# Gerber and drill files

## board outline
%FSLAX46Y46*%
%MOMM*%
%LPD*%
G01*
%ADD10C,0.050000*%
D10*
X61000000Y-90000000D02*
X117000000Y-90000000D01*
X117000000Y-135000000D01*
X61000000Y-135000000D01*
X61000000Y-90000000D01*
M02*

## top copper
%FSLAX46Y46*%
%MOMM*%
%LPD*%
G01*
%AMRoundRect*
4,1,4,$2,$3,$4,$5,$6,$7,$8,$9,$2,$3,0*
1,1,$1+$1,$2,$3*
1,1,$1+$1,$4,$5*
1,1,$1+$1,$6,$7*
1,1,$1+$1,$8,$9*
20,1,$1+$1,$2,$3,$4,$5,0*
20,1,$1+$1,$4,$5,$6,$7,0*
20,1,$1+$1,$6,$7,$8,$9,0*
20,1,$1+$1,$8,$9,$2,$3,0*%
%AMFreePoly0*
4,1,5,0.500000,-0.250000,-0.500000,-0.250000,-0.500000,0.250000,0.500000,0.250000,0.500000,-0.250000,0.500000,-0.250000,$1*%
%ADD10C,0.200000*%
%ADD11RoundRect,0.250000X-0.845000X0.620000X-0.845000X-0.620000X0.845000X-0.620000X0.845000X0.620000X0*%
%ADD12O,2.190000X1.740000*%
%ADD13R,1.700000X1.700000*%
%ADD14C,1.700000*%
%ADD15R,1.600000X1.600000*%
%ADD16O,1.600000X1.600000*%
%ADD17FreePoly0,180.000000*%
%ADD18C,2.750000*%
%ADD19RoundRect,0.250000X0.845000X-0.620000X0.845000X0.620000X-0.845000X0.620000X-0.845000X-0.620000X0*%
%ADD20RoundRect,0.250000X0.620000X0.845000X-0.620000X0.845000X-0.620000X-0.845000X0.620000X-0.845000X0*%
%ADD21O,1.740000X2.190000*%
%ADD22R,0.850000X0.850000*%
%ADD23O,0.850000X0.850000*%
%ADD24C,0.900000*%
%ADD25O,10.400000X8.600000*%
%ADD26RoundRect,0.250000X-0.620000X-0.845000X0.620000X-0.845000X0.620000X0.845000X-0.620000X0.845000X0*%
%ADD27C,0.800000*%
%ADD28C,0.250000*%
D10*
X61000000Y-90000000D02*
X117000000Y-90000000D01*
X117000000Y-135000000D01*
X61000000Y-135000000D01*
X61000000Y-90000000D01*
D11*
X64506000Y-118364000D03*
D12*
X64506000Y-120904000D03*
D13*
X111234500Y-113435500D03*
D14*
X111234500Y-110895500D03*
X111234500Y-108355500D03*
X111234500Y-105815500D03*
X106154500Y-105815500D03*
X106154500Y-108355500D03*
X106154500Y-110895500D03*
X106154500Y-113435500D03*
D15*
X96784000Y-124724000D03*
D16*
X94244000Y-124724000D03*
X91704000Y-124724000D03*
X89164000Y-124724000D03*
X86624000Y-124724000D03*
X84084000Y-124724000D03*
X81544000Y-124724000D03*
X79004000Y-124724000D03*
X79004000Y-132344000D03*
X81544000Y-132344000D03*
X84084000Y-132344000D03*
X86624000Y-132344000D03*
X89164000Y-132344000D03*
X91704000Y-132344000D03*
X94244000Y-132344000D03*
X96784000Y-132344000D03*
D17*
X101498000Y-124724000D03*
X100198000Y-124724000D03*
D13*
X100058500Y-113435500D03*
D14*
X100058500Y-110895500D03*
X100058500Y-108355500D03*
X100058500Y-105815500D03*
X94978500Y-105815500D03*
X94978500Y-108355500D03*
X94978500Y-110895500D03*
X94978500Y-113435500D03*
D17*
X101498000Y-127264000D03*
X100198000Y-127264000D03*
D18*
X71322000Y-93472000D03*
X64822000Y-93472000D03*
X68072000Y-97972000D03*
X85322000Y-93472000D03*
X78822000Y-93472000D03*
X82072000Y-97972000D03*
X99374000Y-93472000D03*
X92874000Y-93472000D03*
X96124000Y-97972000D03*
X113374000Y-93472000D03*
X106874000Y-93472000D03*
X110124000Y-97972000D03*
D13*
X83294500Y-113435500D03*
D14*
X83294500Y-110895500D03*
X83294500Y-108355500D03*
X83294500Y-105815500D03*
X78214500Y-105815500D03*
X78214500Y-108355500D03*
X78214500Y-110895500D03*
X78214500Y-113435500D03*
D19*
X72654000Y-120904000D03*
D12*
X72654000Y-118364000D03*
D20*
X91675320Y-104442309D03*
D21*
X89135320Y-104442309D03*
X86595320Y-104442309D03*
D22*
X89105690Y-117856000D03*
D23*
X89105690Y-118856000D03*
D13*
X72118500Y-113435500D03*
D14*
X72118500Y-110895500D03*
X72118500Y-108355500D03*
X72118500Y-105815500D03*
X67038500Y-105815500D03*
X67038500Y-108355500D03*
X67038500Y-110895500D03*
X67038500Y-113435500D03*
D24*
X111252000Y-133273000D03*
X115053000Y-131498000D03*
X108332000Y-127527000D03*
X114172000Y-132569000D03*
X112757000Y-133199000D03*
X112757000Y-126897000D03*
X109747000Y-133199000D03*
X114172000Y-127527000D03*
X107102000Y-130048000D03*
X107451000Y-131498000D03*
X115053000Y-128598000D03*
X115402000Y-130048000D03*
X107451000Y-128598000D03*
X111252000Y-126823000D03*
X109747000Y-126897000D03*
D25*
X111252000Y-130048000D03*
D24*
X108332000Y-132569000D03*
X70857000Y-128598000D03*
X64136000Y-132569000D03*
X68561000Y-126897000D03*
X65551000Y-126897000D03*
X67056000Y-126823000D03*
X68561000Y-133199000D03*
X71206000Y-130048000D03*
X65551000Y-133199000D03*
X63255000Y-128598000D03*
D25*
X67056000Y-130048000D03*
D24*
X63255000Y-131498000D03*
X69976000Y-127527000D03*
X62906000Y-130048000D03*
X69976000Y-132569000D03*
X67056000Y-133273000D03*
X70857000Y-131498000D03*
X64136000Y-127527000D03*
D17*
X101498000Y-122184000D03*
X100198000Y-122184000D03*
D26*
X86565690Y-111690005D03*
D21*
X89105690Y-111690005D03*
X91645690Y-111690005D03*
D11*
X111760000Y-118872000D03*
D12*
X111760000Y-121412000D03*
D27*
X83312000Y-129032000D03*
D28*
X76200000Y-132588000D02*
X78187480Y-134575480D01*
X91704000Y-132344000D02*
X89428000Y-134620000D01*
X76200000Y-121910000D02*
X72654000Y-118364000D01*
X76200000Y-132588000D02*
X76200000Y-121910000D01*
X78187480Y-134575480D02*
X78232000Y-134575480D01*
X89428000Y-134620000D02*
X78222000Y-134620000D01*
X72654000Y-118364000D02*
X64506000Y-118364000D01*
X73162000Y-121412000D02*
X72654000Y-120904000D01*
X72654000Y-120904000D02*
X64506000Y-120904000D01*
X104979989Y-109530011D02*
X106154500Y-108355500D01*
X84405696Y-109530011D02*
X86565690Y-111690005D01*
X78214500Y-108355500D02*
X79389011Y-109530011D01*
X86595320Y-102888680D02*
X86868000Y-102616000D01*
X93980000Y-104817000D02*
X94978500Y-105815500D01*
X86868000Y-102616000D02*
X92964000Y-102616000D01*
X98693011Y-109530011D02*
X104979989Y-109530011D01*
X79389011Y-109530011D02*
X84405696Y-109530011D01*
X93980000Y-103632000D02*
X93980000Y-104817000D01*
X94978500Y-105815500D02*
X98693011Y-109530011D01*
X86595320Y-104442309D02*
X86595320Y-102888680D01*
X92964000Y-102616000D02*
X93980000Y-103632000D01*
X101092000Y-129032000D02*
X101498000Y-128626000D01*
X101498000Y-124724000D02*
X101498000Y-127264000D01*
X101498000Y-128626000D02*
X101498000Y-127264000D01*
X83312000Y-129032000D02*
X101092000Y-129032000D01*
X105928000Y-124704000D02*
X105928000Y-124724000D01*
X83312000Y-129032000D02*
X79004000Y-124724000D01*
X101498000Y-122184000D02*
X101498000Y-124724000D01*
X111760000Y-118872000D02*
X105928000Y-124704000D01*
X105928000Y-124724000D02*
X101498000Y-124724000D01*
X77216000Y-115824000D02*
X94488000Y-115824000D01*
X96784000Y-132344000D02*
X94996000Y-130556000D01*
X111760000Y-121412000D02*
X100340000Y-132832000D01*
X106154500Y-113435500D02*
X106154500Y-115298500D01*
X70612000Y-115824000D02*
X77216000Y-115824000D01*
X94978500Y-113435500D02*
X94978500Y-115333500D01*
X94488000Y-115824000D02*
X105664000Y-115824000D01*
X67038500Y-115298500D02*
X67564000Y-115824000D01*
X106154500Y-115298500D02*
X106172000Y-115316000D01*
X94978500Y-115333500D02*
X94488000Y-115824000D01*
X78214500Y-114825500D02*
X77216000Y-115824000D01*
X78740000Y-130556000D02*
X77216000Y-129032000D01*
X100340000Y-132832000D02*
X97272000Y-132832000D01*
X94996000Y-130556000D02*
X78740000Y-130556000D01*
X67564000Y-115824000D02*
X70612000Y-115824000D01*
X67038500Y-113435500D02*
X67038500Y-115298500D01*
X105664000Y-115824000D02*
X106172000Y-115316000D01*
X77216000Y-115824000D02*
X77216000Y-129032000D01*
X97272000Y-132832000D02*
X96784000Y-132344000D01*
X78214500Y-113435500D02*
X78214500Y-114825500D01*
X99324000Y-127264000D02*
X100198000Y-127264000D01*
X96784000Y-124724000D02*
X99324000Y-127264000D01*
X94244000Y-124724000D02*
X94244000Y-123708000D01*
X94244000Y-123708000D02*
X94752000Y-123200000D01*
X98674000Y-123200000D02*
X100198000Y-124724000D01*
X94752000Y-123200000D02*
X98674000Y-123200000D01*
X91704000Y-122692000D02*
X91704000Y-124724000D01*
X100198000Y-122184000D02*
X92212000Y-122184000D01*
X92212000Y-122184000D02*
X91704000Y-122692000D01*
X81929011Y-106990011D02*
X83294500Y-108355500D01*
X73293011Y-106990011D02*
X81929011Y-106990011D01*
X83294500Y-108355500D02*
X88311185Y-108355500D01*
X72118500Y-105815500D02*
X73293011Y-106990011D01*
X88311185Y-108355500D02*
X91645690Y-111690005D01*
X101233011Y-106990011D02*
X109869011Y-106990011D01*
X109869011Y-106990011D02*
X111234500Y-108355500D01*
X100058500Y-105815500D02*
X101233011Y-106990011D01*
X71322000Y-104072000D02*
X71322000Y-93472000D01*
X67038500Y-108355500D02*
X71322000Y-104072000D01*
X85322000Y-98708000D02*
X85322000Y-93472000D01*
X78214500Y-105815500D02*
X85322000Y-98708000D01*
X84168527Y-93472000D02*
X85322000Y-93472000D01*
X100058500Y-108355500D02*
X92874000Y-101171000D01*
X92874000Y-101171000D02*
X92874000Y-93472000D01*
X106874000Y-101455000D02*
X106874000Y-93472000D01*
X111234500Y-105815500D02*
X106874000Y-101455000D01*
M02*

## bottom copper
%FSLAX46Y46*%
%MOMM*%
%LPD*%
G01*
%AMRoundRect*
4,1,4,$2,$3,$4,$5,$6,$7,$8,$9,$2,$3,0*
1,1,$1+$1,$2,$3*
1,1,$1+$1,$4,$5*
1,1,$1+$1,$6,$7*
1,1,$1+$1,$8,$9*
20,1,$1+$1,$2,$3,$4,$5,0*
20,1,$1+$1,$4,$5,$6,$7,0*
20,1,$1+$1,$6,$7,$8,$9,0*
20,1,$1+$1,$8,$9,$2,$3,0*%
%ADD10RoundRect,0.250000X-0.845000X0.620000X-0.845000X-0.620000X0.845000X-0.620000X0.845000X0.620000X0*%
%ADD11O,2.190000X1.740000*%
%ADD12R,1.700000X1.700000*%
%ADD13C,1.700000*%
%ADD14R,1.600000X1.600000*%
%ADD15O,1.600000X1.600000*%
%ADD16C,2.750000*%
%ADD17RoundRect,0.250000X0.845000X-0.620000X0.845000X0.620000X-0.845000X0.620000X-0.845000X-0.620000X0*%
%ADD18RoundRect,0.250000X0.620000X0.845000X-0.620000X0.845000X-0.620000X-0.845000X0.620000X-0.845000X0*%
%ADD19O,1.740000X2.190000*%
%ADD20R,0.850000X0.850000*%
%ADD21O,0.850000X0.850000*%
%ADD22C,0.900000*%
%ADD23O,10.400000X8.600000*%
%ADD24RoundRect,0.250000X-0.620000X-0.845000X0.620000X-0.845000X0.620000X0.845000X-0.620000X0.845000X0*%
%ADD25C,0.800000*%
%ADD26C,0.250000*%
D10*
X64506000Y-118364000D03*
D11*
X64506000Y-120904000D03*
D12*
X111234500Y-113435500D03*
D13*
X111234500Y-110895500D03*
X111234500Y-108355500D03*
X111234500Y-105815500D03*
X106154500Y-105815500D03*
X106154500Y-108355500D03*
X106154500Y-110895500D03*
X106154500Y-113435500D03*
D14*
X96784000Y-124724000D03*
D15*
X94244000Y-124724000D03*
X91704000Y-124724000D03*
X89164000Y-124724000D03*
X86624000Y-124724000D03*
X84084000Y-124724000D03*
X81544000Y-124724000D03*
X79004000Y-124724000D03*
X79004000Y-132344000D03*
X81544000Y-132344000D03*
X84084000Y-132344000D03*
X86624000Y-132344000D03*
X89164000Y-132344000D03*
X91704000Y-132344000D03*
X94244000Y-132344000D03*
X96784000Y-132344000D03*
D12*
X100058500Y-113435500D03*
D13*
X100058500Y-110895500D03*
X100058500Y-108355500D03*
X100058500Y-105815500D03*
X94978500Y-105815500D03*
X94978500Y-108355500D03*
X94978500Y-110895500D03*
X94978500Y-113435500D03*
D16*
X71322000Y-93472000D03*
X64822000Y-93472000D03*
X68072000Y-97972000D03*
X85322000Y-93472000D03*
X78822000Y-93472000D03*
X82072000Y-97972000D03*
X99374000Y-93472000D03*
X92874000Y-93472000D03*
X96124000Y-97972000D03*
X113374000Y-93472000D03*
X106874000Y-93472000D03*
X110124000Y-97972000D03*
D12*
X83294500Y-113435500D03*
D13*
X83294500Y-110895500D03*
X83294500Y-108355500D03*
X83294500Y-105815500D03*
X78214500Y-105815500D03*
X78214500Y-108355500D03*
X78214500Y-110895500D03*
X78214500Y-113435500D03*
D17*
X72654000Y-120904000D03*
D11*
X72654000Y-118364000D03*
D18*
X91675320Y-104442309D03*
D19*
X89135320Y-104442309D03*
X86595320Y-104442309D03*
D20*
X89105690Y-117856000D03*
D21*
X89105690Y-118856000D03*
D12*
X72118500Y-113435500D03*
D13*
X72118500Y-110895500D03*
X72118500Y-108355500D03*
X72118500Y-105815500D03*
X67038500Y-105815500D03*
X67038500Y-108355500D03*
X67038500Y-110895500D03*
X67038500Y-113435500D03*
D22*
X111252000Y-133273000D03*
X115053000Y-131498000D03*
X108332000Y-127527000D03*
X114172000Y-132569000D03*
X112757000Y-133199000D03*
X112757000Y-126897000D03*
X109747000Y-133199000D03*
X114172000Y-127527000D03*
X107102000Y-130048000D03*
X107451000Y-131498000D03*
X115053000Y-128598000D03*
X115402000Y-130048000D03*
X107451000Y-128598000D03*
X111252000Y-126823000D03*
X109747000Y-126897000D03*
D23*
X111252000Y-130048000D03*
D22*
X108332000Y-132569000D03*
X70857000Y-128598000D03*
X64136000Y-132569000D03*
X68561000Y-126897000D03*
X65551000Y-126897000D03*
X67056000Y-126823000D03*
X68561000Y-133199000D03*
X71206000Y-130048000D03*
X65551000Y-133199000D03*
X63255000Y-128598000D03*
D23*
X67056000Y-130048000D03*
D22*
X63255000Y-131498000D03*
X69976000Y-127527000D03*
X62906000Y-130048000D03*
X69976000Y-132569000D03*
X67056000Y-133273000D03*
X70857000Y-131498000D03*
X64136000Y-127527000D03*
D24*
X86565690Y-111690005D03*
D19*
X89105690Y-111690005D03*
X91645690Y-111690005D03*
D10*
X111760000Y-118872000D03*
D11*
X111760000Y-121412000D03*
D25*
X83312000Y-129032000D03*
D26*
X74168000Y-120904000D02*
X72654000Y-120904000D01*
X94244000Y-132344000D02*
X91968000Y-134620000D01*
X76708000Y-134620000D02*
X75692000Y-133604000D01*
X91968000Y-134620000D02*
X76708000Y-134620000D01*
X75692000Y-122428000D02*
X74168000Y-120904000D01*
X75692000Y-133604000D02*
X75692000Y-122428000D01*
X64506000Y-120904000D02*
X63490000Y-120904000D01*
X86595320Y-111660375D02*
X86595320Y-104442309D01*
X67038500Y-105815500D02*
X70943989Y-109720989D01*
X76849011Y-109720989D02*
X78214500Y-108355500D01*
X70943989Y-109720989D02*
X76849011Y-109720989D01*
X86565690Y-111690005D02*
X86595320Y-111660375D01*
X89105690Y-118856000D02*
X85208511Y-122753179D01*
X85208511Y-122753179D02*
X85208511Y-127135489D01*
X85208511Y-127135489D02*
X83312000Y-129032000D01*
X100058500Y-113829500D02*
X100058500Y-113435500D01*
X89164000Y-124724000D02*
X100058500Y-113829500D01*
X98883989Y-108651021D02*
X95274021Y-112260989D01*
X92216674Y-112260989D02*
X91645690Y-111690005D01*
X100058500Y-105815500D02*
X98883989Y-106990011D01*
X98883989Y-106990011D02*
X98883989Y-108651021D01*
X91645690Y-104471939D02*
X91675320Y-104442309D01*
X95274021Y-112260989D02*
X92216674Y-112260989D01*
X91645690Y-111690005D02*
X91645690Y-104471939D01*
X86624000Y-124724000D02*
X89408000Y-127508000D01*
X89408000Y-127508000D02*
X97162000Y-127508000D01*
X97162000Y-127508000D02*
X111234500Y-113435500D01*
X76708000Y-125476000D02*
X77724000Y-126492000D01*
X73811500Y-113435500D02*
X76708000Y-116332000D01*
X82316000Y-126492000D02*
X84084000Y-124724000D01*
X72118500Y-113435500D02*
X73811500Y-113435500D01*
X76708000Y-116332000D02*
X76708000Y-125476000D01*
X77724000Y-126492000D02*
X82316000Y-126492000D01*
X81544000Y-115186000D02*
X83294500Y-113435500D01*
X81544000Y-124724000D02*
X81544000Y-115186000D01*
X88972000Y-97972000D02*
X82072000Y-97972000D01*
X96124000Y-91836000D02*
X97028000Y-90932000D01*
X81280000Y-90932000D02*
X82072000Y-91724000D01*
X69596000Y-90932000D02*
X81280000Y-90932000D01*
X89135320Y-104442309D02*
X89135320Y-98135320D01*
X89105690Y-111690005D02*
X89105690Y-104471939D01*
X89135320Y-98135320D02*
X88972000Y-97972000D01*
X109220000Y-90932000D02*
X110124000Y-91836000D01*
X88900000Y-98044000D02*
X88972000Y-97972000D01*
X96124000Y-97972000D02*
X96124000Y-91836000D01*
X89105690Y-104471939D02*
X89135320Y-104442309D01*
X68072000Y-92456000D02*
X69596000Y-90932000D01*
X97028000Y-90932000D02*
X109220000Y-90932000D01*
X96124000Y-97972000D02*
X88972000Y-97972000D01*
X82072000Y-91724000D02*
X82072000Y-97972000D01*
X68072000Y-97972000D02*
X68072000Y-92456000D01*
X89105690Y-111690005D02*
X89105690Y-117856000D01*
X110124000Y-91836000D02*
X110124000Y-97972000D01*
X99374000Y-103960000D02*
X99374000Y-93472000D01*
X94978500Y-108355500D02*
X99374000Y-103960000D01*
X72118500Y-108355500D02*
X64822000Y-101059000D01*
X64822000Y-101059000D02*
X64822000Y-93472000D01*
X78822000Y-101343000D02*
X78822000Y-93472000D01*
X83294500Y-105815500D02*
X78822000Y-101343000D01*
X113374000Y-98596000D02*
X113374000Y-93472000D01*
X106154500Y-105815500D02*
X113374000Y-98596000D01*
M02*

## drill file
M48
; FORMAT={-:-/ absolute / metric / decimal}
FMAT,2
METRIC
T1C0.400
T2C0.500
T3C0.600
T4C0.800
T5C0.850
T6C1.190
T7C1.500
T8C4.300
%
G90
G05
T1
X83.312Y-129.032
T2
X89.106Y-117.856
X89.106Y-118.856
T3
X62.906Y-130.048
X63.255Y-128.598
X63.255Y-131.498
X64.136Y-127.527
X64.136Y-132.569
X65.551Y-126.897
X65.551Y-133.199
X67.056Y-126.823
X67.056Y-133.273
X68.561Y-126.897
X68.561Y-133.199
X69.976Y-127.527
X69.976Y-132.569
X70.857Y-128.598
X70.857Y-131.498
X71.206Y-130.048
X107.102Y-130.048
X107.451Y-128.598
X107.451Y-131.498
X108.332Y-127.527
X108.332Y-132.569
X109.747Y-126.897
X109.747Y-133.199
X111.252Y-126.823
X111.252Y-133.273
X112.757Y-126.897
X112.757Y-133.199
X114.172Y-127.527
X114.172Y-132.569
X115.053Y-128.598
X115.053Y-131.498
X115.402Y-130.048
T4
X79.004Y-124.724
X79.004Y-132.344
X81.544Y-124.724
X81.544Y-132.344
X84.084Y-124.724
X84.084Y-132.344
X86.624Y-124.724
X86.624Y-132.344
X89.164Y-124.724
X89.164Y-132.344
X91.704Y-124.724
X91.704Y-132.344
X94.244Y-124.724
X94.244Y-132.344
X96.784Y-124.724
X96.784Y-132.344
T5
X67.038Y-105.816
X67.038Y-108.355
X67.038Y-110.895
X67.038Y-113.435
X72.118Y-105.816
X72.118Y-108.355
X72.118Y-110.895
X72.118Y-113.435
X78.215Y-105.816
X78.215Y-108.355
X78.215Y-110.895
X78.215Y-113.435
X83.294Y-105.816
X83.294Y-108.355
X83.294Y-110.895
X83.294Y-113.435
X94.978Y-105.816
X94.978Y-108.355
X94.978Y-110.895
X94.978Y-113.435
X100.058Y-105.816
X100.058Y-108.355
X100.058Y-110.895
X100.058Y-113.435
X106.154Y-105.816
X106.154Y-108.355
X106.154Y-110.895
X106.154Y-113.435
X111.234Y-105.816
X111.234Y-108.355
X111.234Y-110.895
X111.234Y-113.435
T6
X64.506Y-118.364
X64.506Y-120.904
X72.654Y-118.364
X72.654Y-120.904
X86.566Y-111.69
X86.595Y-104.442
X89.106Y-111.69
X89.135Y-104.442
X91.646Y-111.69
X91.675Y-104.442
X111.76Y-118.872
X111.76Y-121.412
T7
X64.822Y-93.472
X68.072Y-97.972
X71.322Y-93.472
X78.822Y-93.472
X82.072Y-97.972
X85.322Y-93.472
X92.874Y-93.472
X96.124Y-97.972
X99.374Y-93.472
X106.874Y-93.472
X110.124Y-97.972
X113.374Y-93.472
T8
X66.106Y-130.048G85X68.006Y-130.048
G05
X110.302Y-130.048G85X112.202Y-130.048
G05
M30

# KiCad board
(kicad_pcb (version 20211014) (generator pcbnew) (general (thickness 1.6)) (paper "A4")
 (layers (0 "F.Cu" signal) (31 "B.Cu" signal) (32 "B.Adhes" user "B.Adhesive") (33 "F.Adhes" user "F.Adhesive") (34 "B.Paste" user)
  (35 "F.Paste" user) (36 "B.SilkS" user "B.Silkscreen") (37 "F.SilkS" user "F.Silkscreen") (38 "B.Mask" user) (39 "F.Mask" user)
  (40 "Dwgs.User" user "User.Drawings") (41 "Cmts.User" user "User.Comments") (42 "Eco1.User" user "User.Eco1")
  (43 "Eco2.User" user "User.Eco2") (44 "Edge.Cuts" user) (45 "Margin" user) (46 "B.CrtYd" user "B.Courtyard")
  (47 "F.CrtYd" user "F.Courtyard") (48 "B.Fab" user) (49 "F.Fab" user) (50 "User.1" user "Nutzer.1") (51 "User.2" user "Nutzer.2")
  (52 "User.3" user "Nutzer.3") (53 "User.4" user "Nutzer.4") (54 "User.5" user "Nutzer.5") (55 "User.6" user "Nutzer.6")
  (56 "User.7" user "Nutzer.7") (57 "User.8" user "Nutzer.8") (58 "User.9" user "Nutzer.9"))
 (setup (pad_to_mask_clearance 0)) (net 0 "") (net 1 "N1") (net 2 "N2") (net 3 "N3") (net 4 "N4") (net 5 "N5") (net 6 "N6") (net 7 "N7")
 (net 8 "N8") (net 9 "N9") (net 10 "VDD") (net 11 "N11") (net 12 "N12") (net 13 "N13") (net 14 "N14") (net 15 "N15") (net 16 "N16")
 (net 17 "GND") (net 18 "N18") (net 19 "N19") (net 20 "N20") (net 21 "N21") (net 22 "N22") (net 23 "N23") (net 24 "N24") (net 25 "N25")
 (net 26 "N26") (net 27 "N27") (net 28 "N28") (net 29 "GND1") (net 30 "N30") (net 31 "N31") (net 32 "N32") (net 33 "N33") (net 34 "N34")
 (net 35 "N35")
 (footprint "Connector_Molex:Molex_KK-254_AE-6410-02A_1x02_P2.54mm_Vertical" (layer "F.Cu") (at 64.506 118.364 -90)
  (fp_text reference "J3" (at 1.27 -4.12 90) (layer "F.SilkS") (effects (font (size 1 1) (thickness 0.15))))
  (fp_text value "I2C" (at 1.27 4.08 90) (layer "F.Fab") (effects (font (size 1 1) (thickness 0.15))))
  (pad "1" thru_hole roundrect (at 0 0 270) (size 1.74 2.19) (drill 1.19) (layers *.Cu *.Mask) (roundrect_rratio 0.143678) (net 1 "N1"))
  (pad "2" thru_hole oval (at 2.54 0 270) (size 1.74 2.19) (drill 1.19) (layers *.Cu *.Mask) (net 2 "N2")))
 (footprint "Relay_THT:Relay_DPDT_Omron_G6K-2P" (layer "F.Cu") (at 111.2345 113.4355 180)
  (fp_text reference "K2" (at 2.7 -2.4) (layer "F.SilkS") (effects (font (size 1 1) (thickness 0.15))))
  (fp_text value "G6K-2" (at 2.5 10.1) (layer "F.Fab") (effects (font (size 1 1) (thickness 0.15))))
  (pad "1" thru_hole rect (at 0 0 180) (size 1.7 1.7) (drill 0.85) (layers *.Cu *.Mask) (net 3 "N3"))
  (pad "2" thru_hole circle (at 0 2.54 180) (size 1.7 1.7) (drill 0.85) (layers *.Cu *.Mask) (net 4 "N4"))
  (pad "3" thru_hole circle (at 0 5.08 180) (size 1.7 1.7) (drill 0.85) (layers *.Cu *.Mask) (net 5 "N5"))
  (pad "4" thru_hole circle (at 0 7.62 180) (size 1.7 1.7) (drill 0.85) (layers *.Cu *.Mask) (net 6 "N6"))
  (pad "5" thru_hole circle (at 5.08 7.62 180) (size 1.7 1.7) (drill 0.85) (layers *.Cu *.Mask) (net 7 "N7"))
  (pad "6" thru_hole circle (at 5.08 5.08 180) (size 1.7 1.7) (drill 0.85) (layers *.Cu *.Mask) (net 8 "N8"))
  (pad "7" thru_hole circle (at 5.08 2.54 180) (size 1.7 1.7) (drill 0.85) (layers *.Cu *.Mask) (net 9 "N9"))
  (pad "8" thru_hole circle (at 5.08 0 180) (size 1.7 1.7) (drill 0.85) (layers *.Cu *.Mask) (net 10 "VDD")))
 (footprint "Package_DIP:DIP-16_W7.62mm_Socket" (layer "F.Cu") (at 96.784 124.724 -90)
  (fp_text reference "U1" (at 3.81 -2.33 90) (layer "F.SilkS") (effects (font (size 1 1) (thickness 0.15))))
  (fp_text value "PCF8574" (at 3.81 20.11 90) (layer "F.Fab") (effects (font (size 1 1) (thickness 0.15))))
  (pad "1" thru_hole rect (at 0 0 270) (size 1.6 1.6) (drill 0.8) (layers *.Cu *.Mask) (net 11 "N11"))
  (pad "2" thru_hole oval (at 0 2.54 270) (size 1.6 1.6) (drill 0.8) (layers *.Cu *.Mask) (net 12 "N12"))
  (pad "3" thru_hole oval (at 0 5.08 270) (size 1.6 1.6) (drill 0.8) (layers *.Cu *.Mask) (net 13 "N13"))
  (pad "4" thru_hole oval (at 0 7.62 270) (size 1.6 1.6) (drill 0.8) (layers *.Cu *.Mask) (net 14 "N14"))
  (pad "5" thru_hole oval (at 0 10.16 270) (size 1.6 1.6) (drill 0.8) (layers *.Cu *.Mask) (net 3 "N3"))
  (pad "6" thru_hole oval (at 0 12.7 270) (size 1.6 1.6) (drill 0.8) (layers *.Cu *.Mask) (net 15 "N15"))
  (pad "7" thru_hole oval (at 0 15.24 270) (size 1.6 1.6) (drill 0.8) (layers *.Cu *.Mask) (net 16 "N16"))
  (pad "8" thru_hole oval (at 0 17.78 270) (size 1.6 1.6) (drill 0.8) (layers *.Cu *.Mask) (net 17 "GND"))
  (pad "9" thru_hole oval (at 7.62 17.78 270) (size 1.6 1.6) (drill 0.8) (layers *.Cu *.Mask) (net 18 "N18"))
  (pad "10" thru_hole oval (at 7.62 15.24 270) (size 1.6 1.6) (drill 0.8) (layers *.Cu *.Mask) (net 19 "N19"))
  (pad "11" thru_hole oval (at 7.62 12.7 270) (size 1.6 1.6) (drill 0.8) (layers *.Cu *.Mask) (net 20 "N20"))
  (pad "12" thru_hole oval (at 7.62 10.16 270) (size 1.6 1.6) (drill 0.8) (layers *.Cu *.Mask) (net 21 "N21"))
  (pad "13" thru_hole oval (at 7.62 7.62 270) (size 1.6 1.6) (drill 0.8) (layers *.Cu *.Mask) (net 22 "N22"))
  (pad "14" thru_hole oval (at 7.62 5.08 270) (size 1.6 1.6) (drill 0.8) (layers *.Cu *.Mask) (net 1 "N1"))
  (pad "15" thru_hole oval (at 7.62 2.54 270) (size 1.6 1.6) (drill 0.8) (layers *.Cu *.Mask) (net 2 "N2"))
  (pad "16" thru_hole oval (at 7.62 0 270) (size 1.6 1.6) (drill 0.8) (layers *.Cu *.Mask) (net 10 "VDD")))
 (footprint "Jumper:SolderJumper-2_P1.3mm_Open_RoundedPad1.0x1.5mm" (layer "F.Cu") (at 100.848 124.724 180)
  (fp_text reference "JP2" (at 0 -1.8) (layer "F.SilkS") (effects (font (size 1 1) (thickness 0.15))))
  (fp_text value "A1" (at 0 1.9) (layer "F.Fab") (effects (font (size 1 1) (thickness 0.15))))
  (pad "1" smd custom (at -0.65 0 180) (size 1 0.5) (layers "F.Cu" "F.Mask") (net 17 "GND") (zone_connect 2)
   (options (clearance outline) (anchor rect)) (primitives))
  (pad "2" smd custom (at 0.65 0 180) (size 1 0.5) (layers "F.Cu" "F.Mask") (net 12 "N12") (zone_connect 2)
   (options (clearance outline) (anchor rect)) (primitives)))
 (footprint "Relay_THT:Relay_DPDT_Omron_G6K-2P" (layer "F.Cu") (at 100.0585 113.4355 180)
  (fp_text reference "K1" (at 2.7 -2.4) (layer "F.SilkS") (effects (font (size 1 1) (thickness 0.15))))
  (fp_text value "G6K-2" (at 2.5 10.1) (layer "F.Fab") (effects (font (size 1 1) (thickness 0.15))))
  (pad "1" thru_hole rect (at 0 0 180) (size 1.7 1.7) (drill 0.85) (layers *.Cu *.Mask) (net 14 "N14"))
  (pad "2" thru_hole circle (at 0 2.54 180) (size 1.7 1.7) (drill 0.85) (layers *.Cu *.Mask) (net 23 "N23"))
  (pad "3" thru_hole circle (at 0 5.08 180) (size 1.7 1.7) (drill 0.85) (layers *.Cu *.Mask) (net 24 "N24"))
  (pad "4" thru_hole circle (at 0 7.62 180) (size 1.7 1.7) (drill 0.85) (layers *.Cu *.Mask) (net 5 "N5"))
  (pad "5" thru_hole circle (at 5.08 7.62 180) (size 1.7 1.7) (drill 0.85) (layers *.Cu *.Mask) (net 8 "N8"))
  (pad "6" thru_hole circle (at 5.08 5.08 180) (size 1.7 1.7) (drill 0.85) (layers *.Cu *.Mask) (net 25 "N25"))
  (pad "7" thru_hole circle (at 5.08 2.54 180) (size 1.7 1.7) (drill 0.85) (layers *.Cu *.Mask) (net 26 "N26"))
  (pad "8" thru_hole circle (at 5.08 0 180) (size 1.7 1.7) (drill 0.85) (layers *.Cu *.Mask) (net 10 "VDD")))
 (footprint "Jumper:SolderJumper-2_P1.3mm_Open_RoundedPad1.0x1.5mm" (layer "F.Cu") (at 100.848 127.264 180)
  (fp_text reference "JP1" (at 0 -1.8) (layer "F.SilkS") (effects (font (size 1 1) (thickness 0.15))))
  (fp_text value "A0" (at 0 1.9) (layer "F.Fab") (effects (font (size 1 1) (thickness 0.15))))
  (pad "1" smd custom (at -0.65 0 180) (size 1 0.5) (layers "F.Cu" "F.Mask") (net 17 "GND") (zone_connect 2)
   (options (clearance outline) (anchor rect)) (primitives))
  (pad "2" smd custom (at 0.65 0 180) (size 1 0.5) (layers "F.Cu" "F.Mask") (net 11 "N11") (zone_connect 2)
   (options (clearance outline) (anchor rect)) (primitives)))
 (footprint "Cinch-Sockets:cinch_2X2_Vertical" (layer "F.Cu") (at 68.072 93.472)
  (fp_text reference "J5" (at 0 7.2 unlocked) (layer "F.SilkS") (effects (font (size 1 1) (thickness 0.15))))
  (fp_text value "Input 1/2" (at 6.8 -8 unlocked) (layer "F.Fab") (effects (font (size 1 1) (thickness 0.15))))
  (pad "1" thru_hole circle (at 3.25 0) (size 2.75 2.75) (drill 1.5) (layers *.Cu *.Mask) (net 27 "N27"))
  (pad "2" thru_hole circle (at -3.25 0) (size 2.75 2.75) (drill 1.5) (layers *.Cu *.Mask) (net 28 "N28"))
  (pad "3" thru_hole circle (at 0 4.5) (size 2.75 2.75) (drill 1.5) (layers *.Cu *.Mask) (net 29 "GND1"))
  (pad "4" thru_hole circle (at 17.25 0) (size 2.75 2.75) (drill 1.5) (layers *.Cu *.Mask) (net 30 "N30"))
  (pad "5" thru_hole circle (at 10.75 0) (size 2.75 2.75) (drill 1.5) (layers *.Cu *.Mask) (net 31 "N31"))
  (pad "6" thru_hole circle (at 14 4.5) (size 2.75 2.75) (drill 1.5) (layers *.Cu *.Mask) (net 29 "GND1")))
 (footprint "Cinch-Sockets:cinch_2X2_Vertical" (layer "F.Cu") (at 96.124 93.472)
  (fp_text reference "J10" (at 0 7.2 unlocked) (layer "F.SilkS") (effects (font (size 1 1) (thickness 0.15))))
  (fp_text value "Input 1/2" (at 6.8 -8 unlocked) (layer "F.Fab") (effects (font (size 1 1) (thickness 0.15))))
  (pad "1" thru_hole circle (at 3.25 0) (size 2.75 2.75) (drill 1.5) (layers *.Cu *.Mask) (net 25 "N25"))
  (pad "2" thru_hole circle (at -3.25 0) (size 2.75 2.75) (drill 1.5) (layers *.Cu *.Mask) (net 24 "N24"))
  (pad "3" thru_hole circle (at 0 4.5) (size 2.75 2.75) (drill 1.5) (layers *.Cu *.Mask) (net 29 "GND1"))
  (pad "4" thru_hole circle (at 17.25 0) (size 2.75 2.75) (drill 1.5) (layers *.Cu *.Mask) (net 7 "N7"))
  (pad "5" thru_hole circle (at 10.75 0) (size 2.75 2.75) (drill 1.5) (layers *.Cu *.Mask) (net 6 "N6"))
  (pad "6" thru_hole circle (at 14 4.5) (size 2.75 2.75) (drill 1.5) (layers *.Cu *.Mask) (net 29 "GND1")))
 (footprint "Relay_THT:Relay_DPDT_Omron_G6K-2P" (layer "F.Cu") (at 83.2945 113.4355 180)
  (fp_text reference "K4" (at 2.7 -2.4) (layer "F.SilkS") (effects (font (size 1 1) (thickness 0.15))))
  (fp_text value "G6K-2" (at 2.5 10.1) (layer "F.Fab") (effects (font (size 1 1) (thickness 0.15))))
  (pad "1" thru_hole rect (at 0 0 180) (size 1.7 1.7) (drill 0.85) (layers *.Cu *.Mask) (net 16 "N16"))
  (pad "2" thru_hole circle (at 0 2.54 180) (size 1.7 1.7) (drill 0.85) (layers *.Cu *.Mask) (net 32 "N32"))
  (pad "3" thru_hole circle (at 0 5.08 180) (size 1.7 1.7) (drill 0.85) (layers *.Cu *.Mask) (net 5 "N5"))
  (pad "4" thru_hole circle (at 0 7.62 180) (size 1.7 1.7) (drill 0.85) (layers *.Cu *.Mask) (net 31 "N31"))
  (pad "5" thru_hole circle (at 5.08 7.62 180) (size 1.7 1.7) (drill 0.85) (layers *.Cu *.Mask) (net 30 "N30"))
  (pad "6" thru_hole circle (at 5.08 5.08 180) (size 1.7 1.7) (drill 0.85) (layers *.Cu *.Mask) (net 8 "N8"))
  (pad "7" thru_hole circle (at 5.08 2.54 180) (size 1.7 1.7) (drill 0.85) (layers *.Cu *.Mask) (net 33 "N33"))
  (pad "8" thru_hole circle (at 5.08 0 180) (size 1.7 1.7) (drill 0.85) (layers *.Cu *.Mask) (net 10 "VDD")))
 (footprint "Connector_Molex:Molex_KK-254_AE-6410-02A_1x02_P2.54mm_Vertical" (layer "F.Cu") (at 72.654 120.904 90)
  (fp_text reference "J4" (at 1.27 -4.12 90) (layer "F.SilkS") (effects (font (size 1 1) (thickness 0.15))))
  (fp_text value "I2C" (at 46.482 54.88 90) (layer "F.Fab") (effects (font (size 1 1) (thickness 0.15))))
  (pad "1" thru_hole roundrect (at 0 0 90) (size 1.74 2.19) (drill 1.19) (layers *.Cu *.Mask) (roundrect_rratio 0.143678) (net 2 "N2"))
  (pad "2" thru_hole oval (at 2.54 0 90) (size 1.74 2.19) (drill 1.19) (layers *.Cu *.Mask) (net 1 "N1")))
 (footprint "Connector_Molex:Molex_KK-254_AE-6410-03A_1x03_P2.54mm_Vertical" (layer "F.Cu") (at 91.67532 104.442309 180)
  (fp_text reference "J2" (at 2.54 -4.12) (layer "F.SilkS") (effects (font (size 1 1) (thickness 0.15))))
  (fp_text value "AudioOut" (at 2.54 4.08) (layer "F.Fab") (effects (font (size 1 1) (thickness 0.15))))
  (pad "1" thru_hole roundrect (at 0 0 180) (size 1.74 2.19) (drill 1.19) (layers *.Cu *.Mask) (roundrect_rratio 0.143678) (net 5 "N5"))
  (pad "2" thru_hole oval (at 2.54 0 180) (size 1.74 2.19) (drill 1.19) (layers *.Cu *.Mask) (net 29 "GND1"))
  (pad "3" thru_hole oval (at 5.08 0 180) (size 1.74 2.19) (drill 1.19) (layers *.Cu *.Mask) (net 8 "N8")))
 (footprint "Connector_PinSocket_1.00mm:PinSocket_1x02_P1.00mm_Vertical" (layer "F.Cu") (at 89.10569 117.856)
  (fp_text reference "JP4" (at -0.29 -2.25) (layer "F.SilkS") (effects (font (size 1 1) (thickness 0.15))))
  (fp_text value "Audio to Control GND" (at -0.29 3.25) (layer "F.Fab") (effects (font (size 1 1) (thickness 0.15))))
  (pad "1" thru_hole rect (at 0 0) (size 0.85 0.85) (drill 0.5) (layers *.Cu *.Mask) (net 29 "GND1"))
  (pad "2" thru_hole oval (at 0 1) (size 0.85 0.85) (drill 0.5) (layers *.Cu *.Mask) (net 17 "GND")))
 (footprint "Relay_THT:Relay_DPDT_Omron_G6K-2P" (layer "F.Cu") (at 72.1185 113.4355 180)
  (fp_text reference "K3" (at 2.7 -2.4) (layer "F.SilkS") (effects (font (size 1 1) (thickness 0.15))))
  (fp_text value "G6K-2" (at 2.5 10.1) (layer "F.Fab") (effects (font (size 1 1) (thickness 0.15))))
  (pad "1" thru_hole rect (at 0 0 180) (size 1.7 1.7) (drill 0.85) (layers *.Cu *.Mask) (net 15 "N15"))
  (pad "2" thru_hole circle (at 0 2.54 180) (size 1.7 1.7) (drill 0.85) (layers *.Cu *.Mask) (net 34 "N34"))
  (pad "3" thru_hole circle (at 0 5.08 180) (size 1.7 1.7) (drill 0.85) (layers *.Cu *.Mask) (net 28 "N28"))
  (pad "4" thru_hole circle (at 0 7.62 180) (size 1.7 1.7) (drill 0.85) (layers *.Cu *.Mask) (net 5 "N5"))
  (pad "5" thru_hole circle (at 5.08 7.62 180) (size 1.7 1.7) (drill 0.85) (layers *.Cu *.Mask) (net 8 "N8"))
  (pad "6" thru_hole circle (at 5.08 5.08 180) (size 1.7 1.7) (drill 0.85) (layers *.Cu *.Mask) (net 27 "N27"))
  (pad "7" thru_hole circle (at 5.08 2.54 180) (size 1.7 1.7) (drill 0.85) (layers *.Cu *.Mask) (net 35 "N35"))
  (pad "8" thru_hole circle (at 5.08 0 180) (size 1.7 1.7) (drill 0.85) (layers *.Cu *.Mask) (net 10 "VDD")))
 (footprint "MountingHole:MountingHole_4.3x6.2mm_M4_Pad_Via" (layer "F.Cu") (at 111.252 130.048)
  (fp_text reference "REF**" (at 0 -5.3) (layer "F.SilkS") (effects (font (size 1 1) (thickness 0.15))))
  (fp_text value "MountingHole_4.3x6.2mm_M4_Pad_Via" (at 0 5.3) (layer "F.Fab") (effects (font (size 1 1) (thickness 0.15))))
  (pad "1" thru_hole circle (at 0 3.225) (size 0.9 0.9) (drill 0.6) (layers *.Cu *.Mask))
  (pad "1" thru_hole circle (at 3.801 1.45) (size 0.9 0.9) (drill 0.6) (layers *.Cu *.Mask))
  (pad "1" thru_hole circle (at -2.92 -2.521) (size 0.9 0.9) (drill 0.6) (layers *.Cu *.Mask))
  (pad "1" thru_hole circle (at 2.92 2.521) (size 0.9 0.9) (drill 0.6) (layers *.Cu *.Mask))
  (pad "1" thru_hole circle (at 1.505 3.151) (size 0.9 0.9) (drill 0.6) (layers *.Cu *.Mask))
  (pad "1" thru_hole circle (at 1.505 -3.151) (size 0.9 0.9) (drill 0.6) (layers *.Cu *.Mask))
  (pad "1" thru_hole circle (at -1.505 3.151) (size 0.9 0.9) (drill 0.6) (layers *.Cu *.Mask))
  (pad "1" thru_hole circle (at 2.92 -2.521) (size 0.9 0.9) (drill 0.6) (layers *.Cu *.Mask))
  (pad "1" thru_hole circle (at -4.15 0) (size 0.9 0.9) (drill 0.6) (layers *.Cu *.Mask))
  (pad "1" thru_hole circle (at -3.801 1.45) (size 0.9 0.9) (drill 0.6) (layers *.Cu *.Mask))
  (pad "1" thru_hole circle (at 3.801 -1.45) (size 0.9 0.9) (drill 0.6) (layers *.Cu *.Mask))
  (pad "1" thru_hole circle (at 4.15 0) (size 0.9 0.9) (drill 0.6) (layers *.Cu *.Mask))
  (pad "1" thru_hole circle (at -3.801 -1.45) (size 0.9 0.9) (drill 0.6) (layers *.Cu *.Mask))
  (pad "1" thru_hole circle (at 0 -3.225) (size 0.9 0.9) (drill 0.6) (layers *.Cu *.Mask))
  (pad "1" thru_hole circle (at -1.505 -3.151) (size 0.9 0.9) (drill 0.6) (layers *.Cu *.Mask))
  (pad "1" thru_hole oval (at 0 0) (size 10.4 8.6) (drill oval 6.2 4.3) (layers *.Cu *.Mask))
  (pad "1" thru_hole circle (at -2.92 2.521) (size 0.9 0.9) (drill 0.6) (layers *.Cu *.Mask)))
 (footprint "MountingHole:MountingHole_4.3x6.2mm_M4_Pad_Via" (layer "F.Cu") (at 67.056 130.048)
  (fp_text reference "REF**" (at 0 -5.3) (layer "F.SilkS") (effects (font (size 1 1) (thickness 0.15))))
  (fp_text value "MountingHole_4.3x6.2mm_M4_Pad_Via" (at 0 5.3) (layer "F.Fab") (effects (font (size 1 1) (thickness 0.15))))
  (pad "1" thru_hole circle (at 3.801 -1.45) (size 0.9 0.9) (drill 0.6) (layers *.Cu *.Mask))
  (pad "1" thru_hole circle (at -2.92 2.521) (size 0.9 0.9) (drill 0.6) (layers *.Cu *.Mask))
  (pad "1" thru_hole circle (at 1.505 -3.151) (size 0.9 0.9) (drill 0.6) (layers *.Cu *.Mask))
  (pad "1" thru_hole circle (at -1.505 -3.151) (size 0.9 0.9) (drill 0.6) (layers *.Cu *.Mask))
  (pad "1" thru_hole circle (at 0 -3.225) (size 0.9 0.9) (drill 0.6) (layers *.Cu *.Mask))
  (pad "1" thru_hole circle (at 1.505 3.151) (size 0.9 0.9) (drill 0.6) (layers *.Cu *.Mask))
  (pad "1" thru_hole circle (at 4.15 0) (size 0.9 0.9) (drill 0.6) (layers *.Cu *.Mask))
  (pad "1" thru_hole circle (at -1.505 3.151) (size 0.9 0.9) (drill 0.6) (layers *.Cu *.Mask))
  (pad "1" thru_hole circle (at -3.801 -1.45) (size 0.9 0.9) (drill 0.6) (layers *.Cu *.Mask))
  (pad "1" thru_hole oval (at 0 0) (size 10.4 8.6) (drill oval 6.2 4.3) (layers *.Cu *.Mask))
  (pad "1" thru_hole circle (at -3.801 1.45) (size 0.9 0.9) (drill 0.6) (layers *.Cu *.Mask))
  (pad "1" thru_hole circle (at 2.92 -2.521) (size 0.9 0.9) (drill 0.6) (layers *.Cu *.Mask))
  (pad "1" thru_hole circle (at -4.15 0) (size 0.9 0.9) (drill 0.6) (layers *.Cu *.Mask))
  (pad "1" thru_hole circle (at 2.92 2.521) (size 0.9 0.9) (drill 0.6) (layers *.Cu *.Mask))
  (pad "1" thru_hole circle (at 0 3.225) (size 0.9 0.9) (drill 0.6) (layers *.Cu *.Mask))
  (pad "1" thru_hole circle (at 3.801 1.45) (size 0.9 0.9) (drill 0.6) (layers *.Cu *.Mask))
  (pad "1" thru_hole circle (at -2.92 -2.521) (size 0.9 0.9) (drill 0.6) (layers *.Cu *.Mask)))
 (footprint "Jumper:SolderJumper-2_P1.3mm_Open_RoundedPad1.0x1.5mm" (layer "F.Cu") (at 100.848 122.184 180)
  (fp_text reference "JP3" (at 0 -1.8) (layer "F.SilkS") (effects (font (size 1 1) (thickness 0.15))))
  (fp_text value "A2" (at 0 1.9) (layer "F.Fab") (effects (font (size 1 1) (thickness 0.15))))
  (pad "1" smd custom (at -0.65 0 180) (size 1 0.5) (layers "F.Cu" "F.Mask") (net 17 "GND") (zone_connect 2)
   (options (clearance outline) (anchor rect)) (primitives))
  (pad "2" smd custom (at 0.65 0 180) (size 1 0.5) (layers "F.Cu" "F.Mask") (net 13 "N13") (zone_connect 2)
   (options (clearance outline) (anchor rect)) (primitives)))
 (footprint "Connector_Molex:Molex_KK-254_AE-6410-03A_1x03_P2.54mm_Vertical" (layer "F.Cu") (at 86.56569 111.690005)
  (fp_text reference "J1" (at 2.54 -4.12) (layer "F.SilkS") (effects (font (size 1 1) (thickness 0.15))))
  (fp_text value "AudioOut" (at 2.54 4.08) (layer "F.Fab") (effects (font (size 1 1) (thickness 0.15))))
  (pad "1" thru_hole roundrect (at 0 0) (size 1.74 2.19) (drill 1.19) (layers *.Cu *.Mask) (roundrect_rratio 0.143678) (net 8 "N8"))
  (pad "2" thru_hole oval (at 2.54 0) (size 1.74 2.19) (drill 1.19) (layers *.Cu *.Mask) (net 29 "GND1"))
  (pad "3" thru_hole oval (at 5.08 0) (size 1.74 2.19) (drill 1.19) (layers *.Cu *.Mask) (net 5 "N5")))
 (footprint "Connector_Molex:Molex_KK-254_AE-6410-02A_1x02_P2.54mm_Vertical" (layer "F.Cu") (at 111.76 118.872 -90)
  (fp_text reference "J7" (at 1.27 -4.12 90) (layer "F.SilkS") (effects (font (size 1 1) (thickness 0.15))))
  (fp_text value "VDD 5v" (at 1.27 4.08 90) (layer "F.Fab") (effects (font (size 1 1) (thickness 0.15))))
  (pad "1" thru_hole roundrect (at 0 0 270) (size 1.74 2.19) (drill 1.19) (layers *.Cu *.Mask) (roundrect_rratio 0.143678) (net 17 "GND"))
  (pad "2" thru_hole oval (at 2.54 0 270) (size 1.74 2.19) (drill 1.19) (layers *.Cu *.Mask) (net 10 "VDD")))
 (gr_rect (start 61 90) (end 117 135) (layer "F.Cu") (width 0.2) (fill none))
 (gr_rect (start 61 90) (end 117 135) (layer "Edge.Cuts") (width 0.05) (fill none))
 (segment (start 76.2 132.588) (end 78.18748 134.57548) (width 0.25) (layer "F.Cu") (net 1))
 (segment (start 91.704 132.344) (end 89.428 134.62) (width 0.25) (layer "F.Cu") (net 1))
 (segment (start 76.2 121.91) (end 72.654 118.364) (width 0.25) (layer "F.Cu") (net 1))
 (segment (start 76.2 132.588) (end 76.2 121.91) (width 0.25) (layer "F.Cu") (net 1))
 (segment (start 78.18748 134.57548) (end 78.232 134.57548) (width 0.25) (layer "F.Cu") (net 1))
 (segment (start 89.428 134.62) (end 78.222 134.62) (width 0.25) (layer "F.Cu") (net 1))
 (segment (start 72.654 118.364) (end 64.506 118.364) (width 0.25) (layer "F.Cu") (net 1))
 (segment (start 73.162 121.412) (end 72.654 120.904) (width 0.25) (layer "F.Cu") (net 2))
 (segment (start 72.654 120.904) (end 64.506 120.904) (width 0.25) (layer "F.Cu") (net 2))
 (segment (start 74.168 120.904) (end 72.654 120.904) (width 0.25) (layer "B.Cu") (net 2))
 (segment (start 94.244 132.344) (end 91.968 134.62) (width 0.25) (layer "B.Cu") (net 2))
 (segment (start 76.708 134.62) (end 75.692 133.604) (width 0.25) (layer "B.Cu") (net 2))
 (segment (start 91.968 134.62) (end 76.708 134.62) (width 0.25) (layer "B.Cu") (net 2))
 (segment (start 75.692 122.428) (end 74.168 120.904) (width 0.25) (layer "B.Cu") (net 2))
 (segment (start 75.692 133.604) (end 75.692 122.428) (width 0.25) (layer "B.Cu") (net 2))
 (segment (start 64.506 120.904) (end 63.49 120.904) (width 0.25) (layer "B.Cu") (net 2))
 (segment (start 104.979989 109.530011) (end 106.1545 108.3555) (width 0.25) (layer "F.Cu") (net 8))
 (segment (start 84.405696 109.530011) (end 86.56569 111.690005) (width 0.25) (layer "F.Cu") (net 8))
 (segment (start 78.2145 108.3555) (end 79.389011 109.530011) (width 0.25) (layer "F.Cu") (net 8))
 (segment (start 86.59532 102.88868) (end 86.868 102.616) (width 0.25) (layer "F.Cu") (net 8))
 (segment (start 93.98 104.817) (end 94.9785 105.8155) (width 0.25) (layer "F.Cu") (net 8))
 (segment (start 86.868 102.616) (end 92.964 102.616) (width 0.25) (layer "F.Cu") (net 8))
 (segment (start 98.693011 109.530011) (end 104.979989 109.530011) (width 0.25) (layer "F.Cu") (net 8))
 (segment (start 79.389011 109.530011) (end 84.405696 109.530011) (width 0.25) (layer "F.Cu") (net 8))
 (segment (start 93.98 103.632) (end 93.98 104.817) (width 0.25) (layer "F.Cu") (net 8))
 (segment (start 94.9785 105.8155) (end 98.693011 109.530011) (width 0.25) (layer "F.Cu") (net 8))
 (segment (start 86.59532 104.442309) (end 86.59532 102.88868) (width 0.25) (layer "F.Cu") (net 8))
 (segment (start 92.964 102.616) (end 93.98 103.632) (width 0.25) (layer "F.Cu") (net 8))
 (segment (start 86.59532 111.660375) (end 86.59532 104.442309) (width 0.25) (layer "B.Cu") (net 8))
 (segment (start 67.0385 105.8155) (end 70.943989 109.720989) (width 0.25) (layer "B.Cu") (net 8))
 (segment (start 76.849011 109.720989) (end 78.2145 108.3555) (width 0.25) (layer "B.Cu") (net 8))
 (segment (start 70.943989 109.720989) (end 76.849011 109.720989) (width 0.25) (layer "B.Cu") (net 8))
 (segment (start 86.56569 111.690005) (end 86.59532 111.660375) (width 0.25) (layer "B.Cu") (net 8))
 (segment (start 101.092 129.032) (end 101.498 128.626) (width 0.25) (layer "F.Cu") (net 17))
 (segment (start 101.498 124.724) (end 101.498 127.264) (width 0.25) (layer "F.Cu") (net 17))
 (segment (start 101.498 128.626) (end 101.498 127.264) (width 0.25) (layer "F.Cu") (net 17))
 (segment (start 83.312 129.032) (end 101.092 129.032) (width 0.25) (layer "F.Cu") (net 17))
 (segment (start 105.928 124.704) (end 105.928 124.724) (width 0.25) (layer "F.Cu") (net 17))
 (segment (start 83.312 129.032) (end 79.004 124.724) (width 0.25) (layer "F.Cu") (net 17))
 (segment (start 101.498 122.184) (end 101.498 124.724) (width 0.25) (layer "F.Cu") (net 17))
 (segment (start 111.76 118.872) (end 105.928 124.704) (width 0.25) (layer "F.Cu") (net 17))
 (segment (start 105.928 124.724) (end 101.498 124.724) (width 0.25) (layer "F.Cu") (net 17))
 (via (at 83.312 129.032) (size 0.8) (drill 0.4) (layers "F.Cu" "B.Cu") (free) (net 17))
 (segment (start 89.10569 118.856) (end 85.208511 122.753179) (width 0.25) (layer "B.Cu") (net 17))
 (segment (start 85.208511 122.753179) (end 85.208511 127.135489) (width 0.25) (layer "B.Cu") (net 17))
 (segment (start 85.208511 127.135489) (end 83.312 129.032) (width 0.25) (layer "B.Cu") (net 17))
 (segment (start 77.216 115.824) (end 94.488 115.824) (width 0.25) (layer "F.Cu") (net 10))
 (segment (start 96.784 132.344) (end 94.996 130.556) (width 0.25) (layer "F.Cu") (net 10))
 (segment (start 111.76 121.412) (end 100.34 132.832) (width 0.25) (layer "F.Cu") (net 10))
 (segment (start 106.1545 113.4355) (end 106.1545 115.2985) (width 0.25) (layer "F.Cu") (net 10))
 (segment (start 70.612 115.824) (end 77.216 115.824) (width 0.25) (layer "F.Cu") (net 10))
 (segment (start 94.9785 113.4355) (end 94.9785 115.3335) (width 0.25) (layer "F.Cu") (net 10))
 (segment (start 94.488 115.824) (end 105.664 115.824) (width 0.25) (layer "F.Cu") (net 10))
 (segment (start 67.0385 115.2985) (end 67.564 115.824) (width 0.25) (layer "F.Cu") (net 10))
 (segment (start 106.1545 115.2985) (end 106.172 115.316) (width 0.25) (layer "F.Cu") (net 10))
 (segment (start 94.9785 115.3335) (end 94.488 115.824) (width 0.25) (layer "F.Cu") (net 10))
 (segment (start 78.2145 114.8255) (end 77.216 115.824) (width 0.25) (layer "F.Cu") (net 10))
 (segment (start 78.74 130.556) (end 77.216 129.032) (width 0.25) (layer "F.Cu") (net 10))
 (segment (start 100.34 132.832) (end 97.272 132.832) (width 0.25) (layer "F.Cu") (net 10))
 (segment (start 94.996 130.556) (end 78.74 130.556) (width 0.25) (layer "F.Cu") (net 10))
 (segment (start 67.564 115.824) (end 70.612 115.824) (width 0.25) (layer "F.Cu") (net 10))
 (segment (start 67.0385 113.4355) (end 67.0385 115.2985) (width 0.25) (layer "F.Cu") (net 10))
 (segment (start 105.664 115.824) (end 106.172 115.316) (width 0.25) (layer "F.Cu") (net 10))
 (segment (start 77.216 115.824) (end 77.216 129.032) (width 0.25) (layer "F.Cu") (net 10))
 (segment (start 97.272 132.832) (end 96.784 132.344) (width 0.25) (layer "F.Cu") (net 10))
 (segment (start 78.2145 113.4355) (end 78.2145 114.8255) (width 0.25) (layer "F.Cu") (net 10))
 (segment (start 99.324 127.264) (end 100.198 127.264) (width 0.25) (layer "F.Cu") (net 11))
 (segment (start 96.784 124.724) (end 99.324 127.264) (width 0.25) (layer "F.Cu") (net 11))
 (segment (start 94.244 124.724) (end 94.244 123.708) (width 0.25) (layer "F.Cu") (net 12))
 (segment (start 94.244 123.708) (end 94.752 123.2) (width 0.25) (layer "F.Cu") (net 12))
 (segment (start 98.674 123.2) (end 100.198 124.724) (width 0.25) (layer "F.Cu") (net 12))
 (segment (start 94.752 123.2) (end 98.674 123.2) (width 0.25) (layer "F.Cu") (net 12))
 (segment (start 91.704 122.692) (end 91.704 124.724) (width 0.25) (layer "F.Cu") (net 13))
 (segment (start 100.198 122.184) (end 92.212 122.184) (width 0.25) (layer "F.Cu") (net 13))
 (segment (start 92.212 122.184) (end 91.704 122.692) (width 0.25) (layer "F.Cu") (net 13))
 (segment (start 100.0585 113.8295) (end 100.0585 113.4355) (width 0.25) (layer "B.Cu") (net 14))
 (segment (start 89.164 124.724) (end 100.0585 113.8295) (width 0.25) (layer "B.Cu") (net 14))
 (segment (start 81.929011 106.990011) (end 83.2945 108.3555) (width 0.25) (layer "F.Cu") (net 5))
 (segment (start 73.293011 106.990011) (end 81.929011 106.990011) (width 0.25) (layer "F.Cu") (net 5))
 (segment (start 83.2945 108.3555) (end 88.311185 108.3555) (width 0.25) (layer "F.Cu") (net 5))
 (segment (start 72.1185 105.8155) (end 73.293011 106.990011) (width 0.25) (layer "F.Cu") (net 5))
 (segment (start 88.311185 108.3555) (end 91.64569 111.690005) (width 0.25) (layer "F.Cu") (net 5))
 (segment (start 101.233011 106.990011) (end 109.869011 106.990011) (width 0.25) (layer "F.Cu") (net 5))
 (segment (start 109.869011 106.990011) (end 111.2345 108.3555) (width 0.25) (layer "F.Cu") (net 5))
 (segment (start 100.0585 105.8155) (end 101.233011 106.990011) (width 0.25) (layer "F.Cu") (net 5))
 (segment (start 98.883989 108.651021) (end 95.274021 112.260989) (width 0.25) (layer "B.Cu") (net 5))
 (segment (start 92.216674 112.260989) (end 91.64569 111.690005) (width 0.25) (layer "B.Cu") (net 5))
 (segment (start 100.0585 105.8155) (end 98.883989 106.990011) (width 0.25) (layer "B.Cu") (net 5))
 (segment (start 98.883989 106.990011) (end 98.883989 108.651021) (width 0.25) (layer "B.Cu") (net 5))
 (segment (start 91.64569 104.471939) (end 91.67532 104.442309) (width 0.25) (layer "B.Cu") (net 5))
 (segment (start 95.274021 112.260989) (end 92.216674 112.260989) (width 0.25) (layer "B.Cu") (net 5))
 (segment (start 91.64569 111.690005) (end 91.64569 104.471939) (width 0.25) (layer "B.Cu") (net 5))
 (segment (start 86.624 124.724) (end 89.408 127.508) (width 0.25) (layer "B.Cu") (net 3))
 (segment (start 89.408 127.508) (end 97.162 127.508) (width 0.25) (layer "B.Cu") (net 3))
 (segment (start 97.162 127.508) (end 111.2345 113.4355) (width 0.25) (layer "B.Cu") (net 3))
 (segment (start 76.708 125.476) (end 77.724 126.492) (width 0.25) (layer "B.Cu") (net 15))
 (segment (start 73.8115 113.4355) (end 76.708 116.332) (width 0.25) (layer "B.Cu") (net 15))
 (segment (start 82.316 126.492) (end 84.084 124.724) (width 0.25) (layer "B.Cu") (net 15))
 (segment (start 72.1185 113.4355) (end 73.8115 113.4355) (width 0.25) (layer "B.Cu") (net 15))
 (segment (start 76.708 116.332) (end 76.708 125.476) (width 0.25) (layer "B.Cu") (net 15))
 (segment (start 77.724 126.492) (end 82.316 126.492) (width 0.25) (layer "B.Cu") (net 15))
 (segment (start 81.544 115.186) (end 83.2945 113.4355) (width 0.25) (layer "B.Cu") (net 16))
 (segment (start 81.544 124.724) (end 81.544 115.186) (width 0.25) (layer "B.Cu") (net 16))
 (segment (start 88.972 97.972) (end 82.072 97.972) (width 0.25) (layer "B.Cu") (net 29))
 (segment (start 96.124 91.836) (end 97.028 90.932) (width 0.25) (layer "B.Cu") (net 29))
 (segment (start 81.28 90.932) (end 82.072 91.724) (width 0.25) (layer "B.Cu") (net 29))
 (segment (start 69.596 90.932) (end 81.28 90.932) (width 0.25) (layer "B.Cu") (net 29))
 (segment (start 89.13532 104.442309) (end 89.13532 98.13532) (width 0.25) (layer "B.Cu") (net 29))
 (segment (start 89.10569 111.690005) (end 89.10569 104.471939) (width 0.25) (layer "B.Cu") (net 29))
 (segment (start 89.13532 98.13532) (end 88.972 97.972) (width 0.25) (layer "B.Cu") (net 29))
 (segment (start 109.22 90.932) (end 110.124 91.836) (width 0.25) (layer "B.Cu") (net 29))
 (segment (start 88.9 98.044) (end 88.972 97.972) (width 0.25) (layer "B.Cu") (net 29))
 (segment (start 96.124 97.972) (end 96.124 91.836) (width 0.25) (layer "B.Cu") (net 29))
 (segment (start 89.10569 104.471939) (end 89.13532 104.442309) (width 0.25) (layer "B.Cu") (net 29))
 (segment (start 68.072 92.456) (end 69.596 90.932) (width 0.25) (layer "B.Cu") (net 29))
 (segment (start 97.028 90.932) (end 109.22 90.932) (width 0.25) (layer "B.Cu") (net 29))
 (segment (start 96.124 97.972) (end 88.972 97.972) (width 0.25) (layer "B.Cu") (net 29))
 (segment (start 82.072 91.724) (end 82.072 97.972) (width 0.25) (layer "B.Cu") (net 29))
 (segment (start 68.072 97.972) (end 68.072 92.456) (width 0.25) (layer "B.Cu") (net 29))
 (segment (start 89.10569 111.690005) (end 89.10569 117.856) (width 0.25) (layer "B.Cu") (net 29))
 (segment (start 110.124 91.836) (end 110.124 97.972) (width 0.25) (layer "B.Cu") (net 29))
 (segment (start 99.374 103.96) (end 99.374 93.472) (width 0.25) (layer "B.Cu") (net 25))
 (segment (start 94.9785 108.3555) (end 99.374 103.96) (width 0.25) (layer "B.Cu") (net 25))
 (segment (start 71.322 104.072) (end 71.322 93.472) (width 0.25) (layer "F.Cu") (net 27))
 (segment (start 67.0385 108.3555) (end 71.322 104.072) (width 0.25) (layer "F.Cu") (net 27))
 (segment (start 72.1185 108.3555) (end 64.822 101.059) (width 0.25) (layer "B.Cu") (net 28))
 (segment (start 64.822 101.059) (end 64.822 93.472) (width 0.25) (layer "B.Cu") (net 28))
 (segment (start 85.322 98.708) (end 85.322 93.472) (width 0.25) (layer "F.Cu") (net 30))
 (segment (start 78.2145 105.8155) (end 85.322 98.708) (width 0.25) (layer "F.Cu") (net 30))
 (segment (start 84.168527 93.472) (end 85.322 93.472) (width 0.25) (layer "F.Cu") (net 30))
 (segment (start 78.822 101.343) (end 78.822 93.472) (width 0.25) (layer "B.Cu") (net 31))
 (segment (start 83.2945 105.8155) (end 78.822 101.343) (width 0.25) (layer "B.Cu") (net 31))
 (segment (start 100.0585 108.3555) (end 92.874 101.171) (width 0.25) (layer "F.Cu") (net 24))
 (segment (start 92.874 101.171) (end 92.874 93.472) (width 0.25) (layer "F.Cu") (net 24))
 (segment (start 113.374 98.596) (end 113.374 93.472) (width 0.25) (layer "B.Cu") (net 7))
 (segment (start 106.1545 105.8155) (end 113.374 98.596) (width 0.25) (layer "B.Cu") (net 7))
 (segment (start 106.874 101.455) (end 106.874 93.472) (width 0.25) (layer "F.Cu") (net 6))
 (segment (start 111.2345 105.8155) (end 106.874 101.455) (width 0.25) (layer "F.Cu") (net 6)))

